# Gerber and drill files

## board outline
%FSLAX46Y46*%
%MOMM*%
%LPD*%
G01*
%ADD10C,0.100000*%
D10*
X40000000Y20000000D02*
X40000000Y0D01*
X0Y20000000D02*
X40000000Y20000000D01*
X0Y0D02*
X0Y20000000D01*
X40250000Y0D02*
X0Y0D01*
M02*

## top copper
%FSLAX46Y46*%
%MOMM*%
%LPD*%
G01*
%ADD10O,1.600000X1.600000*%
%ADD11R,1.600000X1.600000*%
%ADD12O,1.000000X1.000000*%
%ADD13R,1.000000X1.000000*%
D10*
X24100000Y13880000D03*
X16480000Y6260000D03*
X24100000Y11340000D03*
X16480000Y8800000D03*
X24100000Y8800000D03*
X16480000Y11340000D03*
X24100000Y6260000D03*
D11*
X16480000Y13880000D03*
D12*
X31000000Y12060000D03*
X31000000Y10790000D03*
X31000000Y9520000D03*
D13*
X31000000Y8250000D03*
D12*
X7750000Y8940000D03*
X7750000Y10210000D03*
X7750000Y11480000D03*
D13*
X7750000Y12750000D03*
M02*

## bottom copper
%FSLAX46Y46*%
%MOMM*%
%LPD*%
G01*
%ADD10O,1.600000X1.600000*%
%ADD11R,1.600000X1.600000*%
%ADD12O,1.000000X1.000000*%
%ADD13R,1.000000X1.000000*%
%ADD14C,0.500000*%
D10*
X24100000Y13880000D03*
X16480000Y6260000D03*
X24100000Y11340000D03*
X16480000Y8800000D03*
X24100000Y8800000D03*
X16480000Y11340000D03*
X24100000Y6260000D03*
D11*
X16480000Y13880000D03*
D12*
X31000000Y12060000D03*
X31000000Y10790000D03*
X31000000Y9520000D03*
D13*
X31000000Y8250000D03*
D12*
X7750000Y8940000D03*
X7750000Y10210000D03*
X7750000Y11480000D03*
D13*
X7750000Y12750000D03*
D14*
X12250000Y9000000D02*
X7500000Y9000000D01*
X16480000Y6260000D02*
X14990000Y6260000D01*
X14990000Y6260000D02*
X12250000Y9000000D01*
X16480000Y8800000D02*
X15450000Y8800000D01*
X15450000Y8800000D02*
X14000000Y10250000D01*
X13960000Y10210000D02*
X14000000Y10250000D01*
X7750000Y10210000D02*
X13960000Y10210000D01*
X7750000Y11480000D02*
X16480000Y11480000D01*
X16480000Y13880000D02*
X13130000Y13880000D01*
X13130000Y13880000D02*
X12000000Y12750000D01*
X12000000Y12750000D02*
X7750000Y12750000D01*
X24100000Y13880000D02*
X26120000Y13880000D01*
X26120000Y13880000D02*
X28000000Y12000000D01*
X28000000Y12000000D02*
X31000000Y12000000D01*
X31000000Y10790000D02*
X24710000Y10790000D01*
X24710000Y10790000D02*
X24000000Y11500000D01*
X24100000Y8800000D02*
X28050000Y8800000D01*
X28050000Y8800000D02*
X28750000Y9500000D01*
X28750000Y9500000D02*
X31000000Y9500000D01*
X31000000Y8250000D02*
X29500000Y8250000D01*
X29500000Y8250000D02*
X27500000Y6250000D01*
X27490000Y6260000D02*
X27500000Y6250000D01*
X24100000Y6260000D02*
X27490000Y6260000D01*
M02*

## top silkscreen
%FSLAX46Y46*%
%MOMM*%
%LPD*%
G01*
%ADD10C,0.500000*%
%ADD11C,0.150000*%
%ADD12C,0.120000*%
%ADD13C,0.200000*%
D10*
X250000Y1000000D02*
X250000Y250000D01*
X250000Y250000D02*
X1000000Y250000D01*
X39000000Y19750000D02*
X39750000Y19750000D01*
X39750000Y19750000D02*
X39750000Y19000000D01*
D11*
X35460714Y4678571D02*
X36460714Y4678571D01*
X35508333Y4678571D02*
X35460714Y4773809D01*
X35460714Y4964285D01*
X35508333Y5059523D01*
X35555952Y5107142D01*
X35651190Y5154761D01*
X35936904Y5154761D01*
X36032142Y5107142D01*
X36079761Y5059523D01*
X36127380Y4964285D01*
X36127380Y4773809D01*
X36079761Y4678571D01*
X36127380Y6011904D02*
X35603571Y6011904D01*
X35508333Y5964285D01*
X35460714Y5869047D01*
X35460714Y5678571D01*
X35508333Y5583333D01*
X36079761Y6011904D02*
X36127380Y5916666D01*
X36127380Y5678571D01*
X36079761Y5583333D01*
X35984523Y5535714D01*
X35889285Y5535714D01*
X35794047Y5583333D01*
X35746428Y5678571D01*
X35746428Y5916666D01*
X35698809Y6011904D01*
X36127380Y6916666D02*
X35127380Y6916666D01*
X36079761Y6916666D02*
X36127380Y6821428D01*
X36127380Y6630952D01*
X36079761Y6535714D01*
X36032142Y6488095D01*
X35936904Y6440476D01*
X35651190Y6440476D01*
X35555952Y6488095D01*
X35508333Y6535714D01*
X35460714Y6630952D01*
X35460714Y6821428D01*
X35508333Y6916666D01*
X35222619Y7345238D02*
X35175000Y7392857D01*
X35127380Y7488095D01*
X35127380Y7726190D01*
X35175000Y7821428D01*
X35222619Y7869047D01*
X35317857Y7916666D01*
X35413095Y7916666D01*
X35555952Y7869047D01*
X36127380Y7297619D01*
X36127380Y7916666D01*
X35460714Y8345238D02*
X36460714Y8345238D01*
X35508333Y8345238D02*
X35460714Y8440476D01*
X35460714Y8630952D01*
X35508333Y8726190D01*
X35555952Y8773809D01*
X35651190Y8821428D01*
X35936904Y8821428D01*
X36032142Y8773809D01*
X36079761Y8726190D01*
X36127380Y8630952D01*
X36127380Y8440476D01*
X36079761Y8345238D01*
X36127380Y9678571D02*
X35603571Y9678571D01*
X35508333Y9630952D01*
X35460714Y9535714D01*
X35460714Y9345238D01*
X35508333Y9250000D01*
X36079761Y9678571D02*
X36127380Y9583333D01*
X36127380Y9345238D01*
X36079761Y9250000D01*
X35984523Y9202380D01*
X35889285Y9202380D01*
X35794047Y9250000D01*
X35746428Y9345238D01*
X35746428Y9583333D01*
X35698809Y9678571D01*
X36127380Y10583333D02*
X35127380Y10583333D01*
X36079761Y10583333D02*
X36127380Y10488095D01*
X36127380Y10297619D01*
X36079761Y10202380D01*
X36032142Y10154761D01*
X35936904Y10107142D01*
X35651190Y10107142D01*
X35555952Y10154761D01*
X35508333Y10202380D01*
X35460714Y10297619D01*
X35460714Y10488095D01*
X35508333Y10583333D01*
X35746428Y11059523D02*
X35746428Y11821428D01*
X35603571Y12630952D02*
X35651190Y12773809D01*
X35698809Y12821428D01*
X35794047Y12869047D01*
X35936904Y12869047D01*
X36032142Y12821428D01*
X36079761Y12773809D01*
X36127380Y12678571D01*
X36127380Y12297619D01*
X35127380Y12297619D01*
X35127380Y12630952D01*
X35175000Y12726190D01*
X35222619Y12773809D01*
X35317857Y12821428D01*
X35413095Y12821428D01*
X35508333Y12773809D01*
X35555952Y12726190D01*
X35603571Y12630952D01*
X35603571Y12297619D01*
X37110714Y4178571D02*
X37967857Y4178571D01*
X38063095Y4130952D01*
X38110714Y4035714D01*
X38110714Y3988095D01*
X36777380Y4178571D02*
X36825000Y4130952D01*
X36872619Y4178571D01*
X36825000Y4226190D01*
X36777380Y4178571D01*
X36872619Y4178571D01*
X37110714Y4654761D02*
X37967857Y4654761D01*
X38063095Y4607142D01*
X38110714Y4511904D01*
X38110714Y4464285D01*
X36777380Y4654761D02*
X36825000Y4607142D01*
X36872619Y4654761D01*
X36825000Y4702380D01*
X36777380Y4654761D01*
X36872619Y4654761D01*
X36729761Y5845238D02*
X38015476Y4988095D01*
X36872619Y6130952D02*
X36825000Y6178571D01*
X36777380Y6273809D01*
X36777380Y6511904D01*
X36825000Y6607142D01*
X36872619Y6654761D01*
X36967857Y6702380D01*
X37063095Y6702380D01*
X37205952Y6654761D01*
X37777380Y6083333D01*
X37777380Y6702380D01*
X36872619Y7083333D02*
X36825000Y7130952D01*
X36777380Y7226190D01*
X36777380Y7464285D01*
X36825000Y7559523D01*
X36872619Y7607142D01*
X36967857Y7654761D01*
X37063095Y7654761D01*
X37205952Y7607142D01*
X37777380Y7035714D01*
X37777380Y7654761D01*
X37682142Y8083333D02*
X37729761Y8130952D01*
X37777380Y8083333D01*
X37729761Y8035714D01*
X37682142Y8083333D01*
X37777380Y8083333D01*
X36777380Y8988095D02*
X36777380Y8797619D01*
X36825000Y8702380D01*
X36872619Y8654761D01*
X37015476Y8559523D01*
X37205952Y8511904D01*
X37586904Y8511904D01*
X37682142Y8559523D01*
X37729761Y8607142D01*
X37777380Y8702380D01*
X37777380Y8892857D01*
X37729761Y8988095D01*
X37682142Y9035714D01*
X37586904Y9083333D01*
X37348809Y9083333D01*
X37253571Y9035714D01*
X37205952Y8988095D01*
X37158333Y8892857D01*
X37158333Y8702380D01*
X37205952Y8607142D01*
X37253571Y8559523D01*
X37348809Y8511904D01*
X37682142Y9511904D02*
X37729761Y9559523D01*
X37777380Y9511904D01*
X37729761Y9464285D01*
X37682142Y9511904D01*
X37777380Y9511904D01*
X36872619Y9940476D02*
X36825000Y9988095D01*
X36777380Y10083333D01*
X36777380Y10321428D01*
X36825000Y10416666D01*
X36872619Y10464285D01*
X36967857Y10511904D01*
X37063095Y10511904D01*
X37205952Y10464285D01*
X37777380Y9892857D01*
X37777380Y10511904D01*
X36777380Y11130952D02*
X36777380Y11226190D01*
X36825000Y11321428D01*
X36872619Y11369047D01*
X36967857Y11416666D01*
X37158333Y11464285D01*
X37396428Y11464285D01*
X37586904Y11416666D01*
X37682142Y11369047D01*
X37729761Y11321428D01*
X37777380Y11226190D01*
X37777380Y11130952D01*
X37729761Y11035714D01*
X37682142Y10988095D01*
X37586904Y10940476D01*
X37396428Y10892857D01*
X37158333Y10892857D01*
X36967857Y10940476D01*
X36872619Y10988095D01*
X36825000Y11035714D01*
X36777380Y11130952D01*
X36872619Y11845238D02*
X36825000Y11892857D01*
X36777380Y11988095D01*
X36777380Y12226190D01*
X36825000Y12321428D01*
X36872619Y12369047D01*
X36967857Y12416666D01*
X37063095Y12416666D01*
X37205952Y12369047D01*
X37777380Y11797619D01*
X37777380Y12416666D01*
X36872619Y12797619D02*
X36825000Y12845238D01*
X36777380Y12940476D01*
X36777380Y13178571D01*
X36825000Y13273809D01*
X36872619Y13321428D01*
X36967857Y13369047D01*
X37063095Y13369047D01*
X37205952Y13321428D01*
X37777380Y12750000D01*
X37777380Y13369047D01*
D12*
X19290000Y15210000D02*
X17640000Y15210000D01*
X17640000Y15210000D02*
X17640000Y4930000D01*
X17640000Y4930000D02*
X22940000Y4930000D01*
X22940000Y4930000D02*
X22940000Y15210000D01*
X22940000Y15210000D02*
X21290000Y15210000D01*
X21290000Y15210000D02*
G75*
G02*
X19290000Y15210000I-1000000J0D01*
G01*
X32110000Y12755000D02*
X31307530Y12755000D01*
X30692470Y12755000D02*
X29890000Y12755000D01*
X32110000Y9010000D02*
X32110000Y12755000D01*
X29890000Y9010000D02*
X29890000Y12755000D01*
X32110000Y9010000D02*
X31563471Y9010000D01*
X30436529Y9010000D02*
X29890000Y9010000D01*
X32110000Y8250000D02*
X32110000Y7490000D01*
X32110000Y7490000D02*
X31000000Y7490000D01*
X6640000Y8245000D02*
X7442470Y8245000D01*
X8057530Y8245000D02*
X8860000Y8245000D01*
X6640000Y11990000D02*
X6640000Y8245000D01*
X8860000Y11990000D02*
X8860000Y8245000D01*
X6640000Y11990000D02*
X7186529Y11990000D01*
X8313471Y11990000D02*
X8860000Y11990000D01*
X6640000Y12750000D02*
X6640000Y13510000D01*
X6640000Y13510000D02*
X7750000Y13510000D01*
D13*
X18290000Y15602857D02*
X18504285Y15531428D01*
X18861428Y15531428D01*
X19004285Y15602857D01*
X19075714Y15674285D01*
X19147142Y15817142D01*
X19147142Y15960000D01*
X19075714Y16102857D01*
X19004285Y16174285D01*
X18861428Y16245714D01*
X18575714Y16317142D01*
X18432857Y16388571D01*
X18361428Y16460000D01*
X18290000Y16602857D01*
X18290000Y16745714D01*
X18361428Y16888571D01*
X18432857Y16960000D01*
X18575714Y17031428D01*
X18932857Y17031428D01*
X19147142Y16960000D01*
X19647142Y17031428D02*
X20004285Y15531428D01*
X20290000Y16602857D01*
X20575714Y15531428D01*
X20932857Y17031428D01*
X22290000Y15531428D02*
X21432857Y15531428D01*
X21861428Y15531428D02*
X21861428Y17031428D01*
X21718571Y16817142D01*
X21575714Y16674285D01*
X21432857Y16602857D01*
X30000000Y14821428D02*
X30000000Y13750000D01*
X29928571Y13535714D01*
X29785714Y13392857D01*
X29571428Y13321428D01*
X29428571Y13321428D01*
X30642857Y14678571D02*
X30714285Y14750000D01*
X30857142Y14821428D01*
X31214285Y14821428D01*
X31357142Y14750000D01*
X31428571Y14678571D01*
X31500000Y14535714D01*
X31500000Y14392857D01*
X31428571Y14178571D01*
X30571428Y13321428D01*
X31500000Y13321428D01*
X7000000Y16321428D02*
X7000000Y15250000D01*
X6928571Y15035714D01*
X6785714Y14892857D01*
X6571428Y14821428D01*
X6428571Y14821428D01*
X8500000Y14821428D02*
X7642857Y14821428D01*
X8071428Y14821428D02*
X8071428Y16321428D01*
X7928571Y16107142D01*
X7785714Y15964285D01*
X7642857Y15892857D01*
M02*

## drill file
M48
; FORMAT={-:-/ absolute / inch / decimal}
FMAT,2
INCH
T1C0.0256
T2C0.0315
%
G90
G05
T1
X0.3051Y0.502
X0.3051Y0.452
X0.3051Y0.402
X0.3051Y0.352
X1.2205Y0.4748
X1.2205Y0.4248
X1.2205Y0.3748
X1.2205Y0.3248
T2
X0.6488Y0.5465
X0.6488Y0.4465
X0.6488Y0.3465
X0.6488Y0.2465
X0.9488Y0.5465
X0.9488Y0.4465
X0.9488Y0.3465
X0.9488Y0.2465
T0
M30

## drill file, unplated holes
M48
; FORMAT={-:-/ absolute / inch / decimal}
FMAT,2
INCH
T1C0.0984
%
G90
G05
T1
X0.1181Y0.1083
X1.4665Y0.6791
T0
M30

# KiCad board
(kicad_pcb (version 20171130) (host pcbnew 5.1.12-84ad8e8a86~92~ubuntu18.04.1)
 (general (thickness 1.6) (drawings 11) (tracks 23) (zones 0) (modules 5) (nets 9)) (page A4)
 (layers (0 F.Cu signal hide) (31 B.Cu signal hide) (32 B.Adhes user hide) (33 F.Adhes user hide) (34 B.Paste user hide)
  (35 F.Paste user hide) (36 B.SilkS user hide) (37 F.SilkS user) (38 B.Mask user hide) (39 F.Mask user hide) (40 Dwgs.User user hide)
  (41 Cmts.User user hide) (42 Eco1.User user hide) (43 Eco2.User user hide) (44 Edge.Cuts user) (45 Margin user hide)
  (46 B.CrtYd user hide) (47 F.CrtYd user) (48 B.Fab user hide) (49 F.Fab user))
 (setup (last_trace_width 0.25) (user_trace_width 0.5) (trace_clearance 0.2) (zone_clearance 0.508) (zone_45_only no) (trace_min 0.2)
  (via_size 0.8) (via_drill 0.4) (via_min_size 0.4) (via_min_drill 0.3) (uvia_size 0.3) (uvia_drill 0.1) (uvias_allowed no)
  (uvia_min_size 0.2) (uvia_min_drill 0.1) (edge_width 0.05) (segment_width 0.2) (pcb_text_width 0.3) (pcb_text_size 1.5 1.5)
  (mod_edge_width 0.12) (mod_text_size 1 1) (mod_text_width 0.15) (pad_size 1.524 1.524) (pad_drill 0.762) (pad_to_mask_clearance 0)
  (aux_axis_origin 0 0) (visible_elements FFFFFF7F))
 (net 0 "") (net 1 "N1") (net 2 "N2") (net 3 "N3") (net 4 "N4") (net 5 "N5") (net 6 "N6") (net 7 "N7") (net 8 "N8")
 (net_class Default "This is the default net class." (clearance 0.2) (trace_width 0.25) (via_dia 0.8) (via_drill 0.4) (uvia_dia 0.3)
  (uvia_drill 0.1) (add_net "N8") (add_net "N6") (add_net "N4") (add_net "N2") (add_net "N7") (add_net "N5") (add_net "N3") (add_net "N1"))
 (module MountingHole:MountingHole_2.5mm (layer F.Cu) (at 37.25 -17.25)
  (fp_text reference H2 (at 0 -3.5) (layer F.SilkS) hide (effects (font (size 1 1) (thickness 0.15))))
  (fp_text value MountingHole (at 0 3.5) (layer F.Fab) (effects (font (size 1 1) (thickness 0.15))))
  (pad 1 np_thru_hole circle (at 0 0) (size 2.5 2.5) (drill 2.5) (layers *.Cu *.Mask)))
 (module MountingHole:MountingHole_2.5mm (layer F.Cu) (at 3 -2.75)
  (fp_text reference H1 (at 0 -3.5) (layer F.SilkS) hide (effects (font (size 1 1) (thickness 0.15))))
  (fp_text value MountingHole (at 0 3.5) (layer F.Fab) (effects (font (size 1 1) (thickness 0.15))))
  (pad 1 np_thru_hole circle (at 0 0) (size 2.5 2.5) (drill 2.5) (layers *.Cu *.Mask)))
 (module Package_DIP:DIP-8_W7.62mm (layer F.Cu) (at 16.48 -13.88)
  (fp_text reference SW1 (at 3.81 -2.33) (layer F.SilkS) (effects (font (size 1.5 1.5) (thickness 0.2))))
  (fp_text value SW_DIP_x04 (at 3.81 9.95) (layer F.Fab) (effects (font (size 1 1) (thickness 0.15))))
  (fp_line (start 2.81 -1.33) (end 1.16 -1.33) (layer F.SilkS) (width 0.12))
  (fp_line (start 1.16 -1.33) (end 1.16 8.95) (layer F.SilkS) (width 0.12))
  (fp_line (start 1.16 8.95) (end 6.46 8.95) (layer F.SilkS) (width 0.12))
  (fp_line (start 6.46 8.95) (end 6.46 -1.33) (layer F.SilkS) (width 0.12))
  (fp_line (start 6.46 -1.33) (end 4.81 -1.33) (layer F.SilkS) (width 0.12))
  (fp_arc (start 3.81 -1.33) (end 2.81 -1.33) (angle -180) (layer F.SilkS) (width 0.12))
  (pad 8 thru_hole oval (at 7.62 0) (size 1.6 1.6) (drill 0.8) (layers *.Cu *.Mask) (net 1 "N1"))
  (pad 4 thru_hole oval (at 0 7.62) (size 1.6 1.6) (drill 0.8) (layers *.Cu *.Mask) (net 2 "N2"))
  (pad 7 thru_hole oval (at 7.62 2.54) (size 1.6 1.6) (drill 0.8) (layers *.Cu *.Mask) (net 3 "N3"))
  (pad 3 thru_hole oval (at 0 5.08) (size 1.6 1.6) (drill 0.8) (layers *.Cu *.Mask) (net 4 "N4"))
  (pad 6 thru_hole oval (at 7.62 5.08) (size 1.6 1.6) (drill 0.8) (layers *.Cu *.Mask) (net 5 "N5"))
  (pad 2 thru_hole oval (at 0 2.54) (size 1.6 1.6) (drill 0.8) (layers *.Cu *.Mask) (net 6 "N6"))
  (pad 5 thru_hole oval (at 7.62 7.62) (size 1.6 1.6) (drill 0.8) (layers *.Cu *.Mask) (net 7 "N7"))
  (pad 1 thru_hole rect (at 0 0) (size 1.6 1.6) (drill 0.8) (layers *.Cu *.Mask) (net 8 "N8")))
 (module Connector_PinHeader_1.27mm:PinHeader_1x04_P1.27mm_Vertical (layer F.Cu) (at 31 -8.25 180)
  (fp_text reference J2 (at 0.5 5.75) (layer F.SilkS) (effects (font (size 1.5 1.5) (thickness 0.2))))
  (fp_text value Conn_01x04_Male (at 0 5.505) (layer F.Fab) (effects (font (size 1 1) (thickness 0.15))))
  (fp_line (start -1.11 4.505) (end -0.30753 4.505) (layer F.SilkS) (width 0.12))
  (fp_line (start 0.30753 4.505) (end 1.11 4.505) (layer F.SilkS) (width 0.12))
  (fp_line (start -1.11 0.76) (end -1.11 4.505) (layer F.SilkS) (width 0.12))
  (fp_line (start 1.11 0.76) (end 1.11 4.505) (layer F.SilkS) (width 0.12))
  (fp_line (start -1.11 0.76) (end -0.563471 0.76) (layer F.SilkS) (width 0.12))
  (fp_line (start 0.563471 0.76) (end 1.11 0.76) (layer F.SilkS) (width 0.12))
  (fp_line (start -1.11 0) (end -1.11 -0.76) (layer F.SilkS) (width 0.12))
  (fp_line (start -1.11 -0.76) (end 0 -0.76) (layer F.SilkS) (width 0.12))
  (pad 4 thru_hole oval (at 0 3.81 180) (size 1 1) (drill 0.65) (layers *.Cu *.Mask) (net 1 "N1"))
  (pad 3 thru_hole oval (at 0 2.54 180) (size 1 1) (drill 0.65) (layers *.Cu *.Mask) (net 3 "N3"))
  (pad 2 thru_hole oval (at 0 1.27 180) (size 1 1) (drill 0.65) (layers *.Cu *.Mask) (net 5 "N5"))
  (pad 1 thru_hole rect (at 0 0 180) (size 1 1) (drill 0.65) (layers *.Cu *.Mask) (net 7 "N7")))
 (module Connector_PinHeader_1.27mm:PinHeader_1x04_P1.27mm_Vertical (layer F.Cu) (at 7.75 -12.75)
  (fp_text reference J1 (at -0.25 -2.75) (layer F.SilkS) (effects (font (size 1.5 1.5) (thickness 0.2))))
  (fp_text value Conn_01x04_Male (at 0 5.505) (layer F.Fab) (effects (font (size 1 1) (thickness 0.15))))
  (fp_line (start -1.11 4.505) (end -0.30753 4.505) (layer F.SilkS) (width 0.12))
  (fp_line (start 0.30753 4.505) (end 1.11 4.505) (layer F.SilkS) (width 0.12))
  (fp_line (start -1.11 0.76) (end -1.11 4.505) (layer F.SilkS) (width 0.12))
  (fp_line (start 1.11 0.76) (end 1.11 4.505) (layer F.SilkS) (width 0.12))
  (fp_line (start -1.11 0.76) (end -0.563471 0.76) (layer F.SilkS) (width 0.12))
  (fp_line (start 0.563471 0.76) (end 1.11 0.76) (layer F.SilkS) (width 0.12))
  (fp_line (start -1.11 0) (end -1.11 -0.76) (layer F.SilkS) (width 0.12))
  (fp_line (start -1.11 -0.76) (end 0 -0.76) (layer F.SilkS) (width 0.12))
  (pad 4 thru_hole oval (at 0 3.81) (size 1 1) (drill 0.65) (layers *.Cu *.Mask) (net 2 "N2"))
  (pad 3 thru_hole oval (at 0 2.54) (size 1 1) (drill 0.65) (layers *.Cu *.Mask) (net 4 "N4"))
  (pad 2 thru_hole oval (at 0 1.27) (size 1 1) (drill 0.65) (layers *.Cu *.Mask) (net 6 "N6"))
  (pad 1 thru_hole rect (at 0 0) (size 1 1) (drill 0.65) (layers *.Cu *.Mask) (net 8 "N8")))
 (gr_line (start 0.25 -1) (end 0.25 -0.25) (layer F.SilkS) (width 0.5))
 (gr_line (start 0.25 -0.25) (end 1 -0.25) (layer F.SilkS) (width 0.5))
 (gr_line (start 39 -19.75) (end 39.75 -19.75) (layer F.SilkS) (width 0.5))
 (gr_line (start 39.75 -19.75) (end 39.75 -19) (layer F.SilkS) (width 0.5))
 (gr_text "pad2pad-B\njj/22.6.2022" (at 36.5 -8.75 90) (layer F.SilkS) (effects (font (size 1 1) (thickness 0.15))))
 (gr_line (start 40 -20) (end 40 0) (layer Edge.Cuts) (width 0.1))
 (gr_line (start 0 -20) (end 40 -20) (layer Edge.Cuts) (width 0.1))
 (gr_line (start 0 0) (end 0 -20) (layer Edge.Cuts) (width 0.1))
 (gr_line (start 40.25 0) (end 0 0) (layer Edge.Cuts) (width 0.1))
 (segment (start 12.25 -9) (end 7.5 -9) (width 0.5) (layer B.Cu) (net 2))
 (segment (start 16.48 -6.26) (end 14.99 -6.26) (width 0.5) (layer B.Cu) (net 2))
 (segment (start 14.99 -6.26) (end 12.25 -9) (width 0.5) (layer B.Cu) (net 2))
 (segment (start 16.48 -8.8) (end 15.45 -8.8) (width 0.5) (layer B.Cu) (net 4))
 (segment (start 15.45 -8.8) (end 14 -10.25) (width 0.5) (layer B.Cu) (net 4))
 (segment (start 13.96 -10.21) (end 14 -10.25) (width 0.5) (layer B.Cu) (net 4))
 (segment (start 7.75 -10.21) (end 13.96 -10.21) (width 0.5) (layer B.Cu) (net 4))
 (segment (start 7.75 -11.48) (end 16.48 -11.48) (width 0.5) (layer B.Cu) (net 6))
 (segment (start 16.48 -13.88) (end 13.13 -13.88) (width 0.5) (layer B.Cu) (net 8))
 (segment (start 13.13 -13.88) (end 12 -12.75) (width 0.5) (layer B.Cu) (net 8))
 (segment (start 12 -12.75) (end 7.75 -12.75) (width 0.5) (layer B.Cu) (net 8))
 (segment (start 24.1 -13.88) (end 26.12 -13.88) (width 0.5) (layer B.Cu) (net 1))
 (segment (start 26.12 -13.88) (end 28 -12) (width 0.5) (layer B.Cu) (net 1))
 (segment (start 28 -12) (end 31 -12) (width 0.5) (layer B.Cu) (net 1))
 (segment (start 31 -10.79) (end 24.71 -10.79) (width 0.5) (layer B.Cu) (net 3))
 (segment (start 24.71 -10.79) (end 24 -11.5) (width 0.5) (layer B.Cu) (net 3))
 (segment (start 24.1 -8.8) (end 28.05 -8.8) (width 0.5) (layer B.Cu) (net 5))
 (segment (start 28.05 -8.8) (end 28.75 -9.5) (width 0.5) (layer B.Cu) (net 5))
 (segment (start 28.75 -9.5) (end 31 -9.5) (width 0.5) (layer B.Cu) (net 5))
 (segment (start 31 -8.25) (end 29.5 -8.25) (width 0.5) (layer B.Cu) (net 7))
 (segment (start 29.5 -8.25) (end 27.5 -6.25) (width 0.5) (layer B.Cu) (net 7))
 (segment (start 27.49 -6.26) (end 27.5 -6.25) (width 0.5) (layer B.Cu) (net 7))
 (segment (start 24.1 -6.26) (end 27.49 -6.26) (width 0.5) (layer B.Cu) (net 7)))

